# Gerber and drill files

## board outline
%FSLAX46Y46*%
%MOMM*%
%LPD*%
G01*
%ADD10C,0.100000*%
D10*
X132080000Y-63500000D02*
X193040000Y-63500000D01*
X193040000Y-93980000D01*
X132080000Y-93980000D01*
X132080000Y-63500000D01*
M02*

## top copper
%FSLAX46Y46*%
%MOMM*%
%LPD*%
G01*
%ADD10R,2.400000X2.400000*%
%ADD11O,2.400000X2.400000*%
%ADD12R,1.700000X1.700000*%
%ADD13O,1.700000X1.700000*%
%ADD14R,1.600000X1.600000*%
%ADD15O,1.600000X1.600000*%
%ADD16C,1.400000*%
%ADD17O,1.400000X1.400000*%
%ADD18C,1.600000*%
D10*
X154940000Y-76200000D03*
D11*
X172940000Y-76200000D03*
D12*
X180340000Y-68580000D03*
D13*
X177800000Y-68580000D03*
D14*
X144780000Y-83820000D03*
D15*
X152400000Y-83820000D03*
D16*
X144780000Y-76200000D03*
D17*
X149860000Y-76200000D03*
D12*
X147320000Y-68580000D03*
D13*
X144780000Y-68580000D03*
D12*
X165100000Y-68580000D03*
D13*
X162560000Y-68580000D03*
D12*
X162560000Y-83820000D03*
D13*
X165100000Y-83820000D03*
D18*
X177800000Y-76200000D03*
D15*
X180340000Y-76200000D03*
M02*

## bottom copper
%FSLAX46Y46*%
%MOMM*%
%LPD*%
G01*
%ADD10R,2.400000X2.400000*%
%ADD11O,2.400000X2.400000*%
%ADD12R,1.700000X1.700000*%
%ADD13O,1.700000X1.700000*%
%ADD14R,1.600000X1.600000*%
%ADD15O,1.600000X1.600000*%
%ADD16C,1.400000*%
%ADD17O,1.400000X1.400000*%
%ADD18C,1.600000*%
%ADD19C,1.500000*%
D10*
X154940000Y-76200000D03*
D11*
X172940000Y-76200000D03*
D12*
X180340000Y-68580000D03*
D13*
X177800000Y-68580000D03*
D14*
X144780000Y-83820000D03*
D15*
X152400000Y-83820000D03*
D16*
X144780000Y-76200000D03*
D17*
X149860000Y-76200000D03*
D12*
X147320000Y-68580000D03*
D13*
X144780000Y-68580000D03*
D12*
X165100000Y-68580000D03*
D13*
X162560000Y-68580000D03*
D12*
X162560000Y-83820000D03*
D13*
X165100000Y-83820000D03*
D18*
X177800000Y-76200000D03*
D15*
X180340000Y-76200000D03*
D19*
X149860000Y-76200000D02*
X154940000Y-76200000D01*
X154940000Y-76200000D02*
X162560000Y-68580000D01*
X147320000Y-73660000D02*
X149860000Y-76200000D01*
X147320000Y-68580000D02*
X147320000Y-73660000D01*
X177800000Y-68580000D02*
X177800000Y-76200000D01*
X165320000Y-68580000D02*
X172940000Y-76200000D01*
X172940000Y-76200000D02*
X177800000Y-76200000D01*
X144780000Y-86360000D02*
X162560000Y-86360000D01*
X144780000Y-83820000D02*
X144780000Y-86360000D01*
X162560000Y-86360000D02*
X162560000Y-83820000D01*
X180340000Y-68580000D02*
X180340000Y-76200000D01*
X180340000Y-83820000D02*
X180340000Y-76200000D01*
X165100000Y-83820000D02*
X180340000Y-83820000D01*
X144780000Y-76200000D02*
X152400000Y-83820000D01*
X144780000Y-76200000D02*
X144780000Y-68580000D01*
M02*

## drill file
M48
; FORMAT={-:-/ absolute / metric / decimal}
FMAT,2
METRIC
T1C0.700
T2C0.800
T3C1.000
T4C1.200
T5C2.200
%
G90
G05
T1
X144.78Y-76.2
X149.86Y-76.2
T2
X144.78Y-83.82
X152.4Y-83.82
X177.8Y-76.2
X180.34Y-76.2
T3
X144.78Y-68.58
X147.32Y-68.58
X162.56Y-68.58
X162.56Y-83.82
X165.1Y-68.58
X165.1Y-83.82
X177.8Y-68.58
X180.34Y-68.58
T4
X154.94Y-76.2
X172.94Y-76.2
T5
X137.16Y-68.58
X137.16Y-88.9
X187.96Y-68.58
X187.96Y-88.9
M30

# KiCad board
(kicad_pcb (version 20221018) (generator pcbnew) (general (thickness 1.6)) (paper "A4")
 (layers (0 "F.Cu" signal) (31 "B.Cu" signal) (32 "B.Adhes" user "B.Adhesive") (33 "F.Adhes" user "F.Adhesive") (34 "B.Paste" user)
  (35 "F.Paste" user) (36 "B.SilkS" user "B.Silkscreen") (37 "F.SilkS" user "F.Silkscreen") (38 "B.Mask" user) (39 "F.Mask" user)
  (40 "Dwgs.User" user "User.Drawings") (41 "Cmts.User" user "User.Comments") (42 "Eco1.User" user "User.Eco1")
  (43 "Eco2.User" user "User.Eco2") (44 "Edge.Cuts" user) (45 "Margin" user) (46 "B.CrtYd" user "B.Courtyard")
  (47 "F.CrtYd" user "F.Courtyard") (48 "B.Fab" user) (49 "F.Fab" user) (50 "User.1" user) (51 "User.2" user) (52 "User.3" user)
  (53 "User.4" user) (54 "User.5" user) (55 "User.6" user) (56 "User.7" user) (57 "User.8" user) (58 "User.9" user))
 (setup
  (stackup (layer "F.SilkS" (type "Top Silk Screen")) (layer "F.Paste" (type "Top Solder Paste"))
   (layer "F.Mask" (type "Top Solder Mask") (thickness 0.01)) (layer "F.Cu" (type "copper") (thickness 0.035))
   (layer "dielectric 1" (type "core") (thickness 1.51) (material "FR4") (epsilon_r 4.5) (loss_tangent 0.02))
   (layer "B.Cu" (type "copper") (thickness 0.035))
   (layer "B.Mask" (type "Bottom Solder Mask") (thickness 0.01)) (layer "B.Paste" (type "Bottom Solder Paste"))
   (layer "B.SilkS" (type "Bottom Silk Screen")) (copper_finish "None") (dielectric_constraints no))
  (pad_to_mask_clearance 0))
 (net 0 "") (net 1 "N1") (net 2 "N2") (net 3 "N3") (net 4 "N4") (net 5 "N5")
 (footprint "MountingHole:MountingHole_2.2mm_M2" (layer "F.Cu") (at 187.96 68.58)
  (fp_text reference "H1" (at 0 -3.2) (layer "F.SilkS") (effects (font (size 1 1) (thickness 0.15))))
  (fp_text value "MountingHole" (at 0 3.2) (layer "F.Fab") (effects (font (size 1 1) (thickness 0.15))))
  (pad "" np_thru_hole circle (at 0 0) (size 2.2 2.2) (drill 2.2) (layers "*.Cu" "*.Mask")))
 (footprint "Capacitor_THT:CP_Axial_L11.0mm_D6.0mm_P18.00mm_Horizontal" (layer "F.Cu") (at 154.94 76.2)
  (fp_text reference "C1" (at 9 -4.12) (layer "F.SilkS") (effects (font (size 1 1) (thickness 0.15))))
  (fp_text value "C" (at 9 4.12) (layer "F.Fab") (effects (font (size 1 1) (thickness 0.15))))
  (pad "1" thru_hole rect (at 0 0) (size 2.4 2.4) (drill 1.2) (layers "*.Cu" "*.Mask") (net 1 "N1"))
  (pad "2" thru_hole oval (at 18 0) (size 2.4 2.4) (drill 1.2) (layers "*.Cu" "*.Mask") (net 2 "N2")))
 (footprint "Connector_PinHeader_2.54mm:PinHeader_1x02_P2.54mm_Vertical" (layer "F.Cu") (at 180.34 68.58 -90)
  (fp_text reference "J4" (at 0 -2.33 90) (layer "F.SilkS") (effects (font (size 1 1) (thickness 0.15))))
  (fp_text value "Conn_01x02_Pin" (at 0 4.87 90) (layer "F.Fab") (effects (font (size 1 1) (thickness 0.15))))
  (pad "1" thru_hole rect (at 0 0 270) (size 1.7 1.7) (drill 1) (layers "*.Cu" "*.Mask") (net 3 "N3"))
  (pad "2" thru_hole oval (at 0 2.54 270) (size 1.7 1.7) (drill 1) (layers "*.Cu" "*.Mask") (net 2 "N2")))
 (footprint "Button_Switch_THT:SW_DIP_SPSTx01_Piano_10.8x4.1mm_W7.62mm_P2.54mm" (layer "F.Cu") (at 144.78 83.82)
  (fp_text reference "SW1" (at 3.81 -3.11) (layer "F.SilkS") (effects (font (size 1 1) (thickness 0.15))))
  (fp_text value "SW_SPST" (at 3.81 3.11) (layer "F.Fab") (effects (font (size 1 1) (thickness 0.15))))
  (pad "1" thru_hole rect (at 0 0) (size 1.6 1.6) (drill 0.8) (layers "*.Cu" "*.Mask") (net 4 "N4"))
  (pad "2" thru_hole oval (at 7.62 0) (size 1.6 1.6) (drill 0.8) (layers "*.Cu" "*.Mask") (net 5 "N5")))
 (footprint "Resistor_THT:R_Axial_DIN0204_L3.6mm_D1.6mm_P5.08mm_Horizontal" (layer "F.Cu") (at 144.78 76.2)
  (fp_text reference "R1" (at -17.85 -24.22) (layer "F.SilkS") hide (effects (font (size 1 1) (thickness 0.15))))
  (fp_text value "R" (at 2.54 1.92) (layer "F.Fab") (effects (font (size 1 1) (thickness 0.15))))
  (pad "1" thru_hole circle (at 0 0) (size 1.4 1.4) (drill 0.7) (layers "*.Cu" "*.Mask") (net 5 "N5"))
  (pad "2" thru_hole oval (at 5.08 0) (size 1.4 1.4) (drill 0.7) (layers "*.Cu" "*.Mask") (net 1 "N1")))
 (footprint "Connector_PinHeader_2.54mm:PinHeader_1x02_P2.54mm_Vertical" (layer "F.Cu") (at 147.32 68.58 -90)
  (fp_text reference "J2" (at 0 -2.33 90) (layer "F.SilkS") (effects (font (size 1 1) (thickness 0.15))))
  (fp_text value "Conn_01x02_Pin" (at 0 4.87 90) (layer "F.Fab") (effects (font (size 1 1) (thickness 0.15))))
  (pad "1" thru_hole rect (at 0 0 270) (size 1.7 1.7) (drill 1) (layers "*.Cu" "*.Mask") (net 1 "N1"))
  (pad "2" thru_hole oval (at 0 2.54 270) (size 1.7 1.7) (drill 1) (layers "*.Cu" "*.Mask") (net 5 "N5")))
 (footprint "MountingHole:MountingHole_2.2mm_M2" (layer "F.Cu") (at 187.96 88.9)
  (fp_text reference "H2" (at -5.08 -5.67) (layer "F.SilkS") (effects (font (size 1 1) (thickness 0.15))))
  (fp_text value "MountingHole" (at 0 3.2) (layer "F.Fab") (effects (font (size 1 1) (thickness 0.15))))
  (pad "" np_thru_hole circle (at 0 0) (size 2.2 2.2) (drill 2.2) (layers "*.Cu" "*.Mask")))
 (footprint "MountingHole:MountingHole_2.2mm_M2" (layer "F.Cu") (at 137.16 68.58)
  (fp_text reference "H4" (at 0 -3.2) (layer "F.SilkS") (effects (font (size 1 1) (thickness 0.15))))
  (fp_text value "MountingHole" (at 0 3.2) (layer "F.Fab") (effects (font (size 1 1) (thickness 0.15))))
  (pad "" np_thru_hole circle (at 0 0) (size 2.2 2.2) (drill 2.2) (layers "*.Cu" "*.Mask")))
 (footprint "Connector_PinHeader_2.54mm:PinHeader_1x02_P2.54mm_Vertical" (layer "F.Cu") (at 165.1 68.58 -90)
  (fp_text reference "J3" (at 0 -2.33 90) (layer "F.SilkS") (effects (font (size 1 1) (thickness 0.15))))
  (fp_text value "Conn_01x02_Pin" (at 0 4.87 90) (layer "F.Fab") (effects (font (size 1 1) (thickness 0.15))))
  (pad "1" thru_hole rect (at 0 0 270) (size 1.7 1.7) (drill 1) (layers "*.Cu" "*.Mask") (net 2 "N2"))
  (pad "2" thru_hole oval (at 0 2.54 270) (size 1.7 1.7) (drill 1) (layers "*.Cu" "*.Mask") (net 1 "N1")))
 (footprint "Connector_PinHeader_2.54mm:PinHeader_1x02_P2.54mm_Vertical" (layer "F.Cu") (at 162.56 83.82 90)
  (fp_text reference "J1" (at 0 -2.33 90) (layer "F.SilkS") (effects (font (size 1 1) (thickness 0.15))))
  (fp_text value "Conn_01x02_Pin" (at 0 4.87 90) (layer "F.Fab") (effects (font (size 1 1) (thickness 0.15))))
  (pad "1" thru_hole rect (at 0 0 90) (size 1.7 1.7) (drill 1) (layers "*.Cu" "*.Mask") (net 4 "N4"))
  (pad "2" thru_hole oval (at 0 2.54 90) (size 1.7 1.7) (drill 1) (layers "*.Cu" "*.Mask") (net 3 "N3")))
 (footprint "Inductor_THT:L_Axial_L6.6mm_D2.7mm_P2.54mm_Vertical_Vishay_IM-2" (layer "F.Cu") (at 177.8 76.2)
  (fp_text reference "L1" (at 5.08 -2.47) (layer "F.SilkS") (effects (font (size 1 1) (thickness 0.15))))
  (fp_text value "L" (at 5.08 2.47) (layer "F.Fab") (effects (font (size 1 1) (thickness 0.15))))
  (pad "1" thru_hole circle (at 0 0) (size 1.6 1.6) (drill 0.8) (layers "*.Cu" "*.Mask") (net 2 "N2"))
  (pad "2" thru_hole oval (at 2.54 0) (size 1.6 1.6) (drill 0.8) (layers "*.Cu" "*.Mask") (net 3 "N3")))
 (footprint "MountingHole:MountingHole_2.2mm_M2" (layer "F.Cu") (at 137.16 88.9)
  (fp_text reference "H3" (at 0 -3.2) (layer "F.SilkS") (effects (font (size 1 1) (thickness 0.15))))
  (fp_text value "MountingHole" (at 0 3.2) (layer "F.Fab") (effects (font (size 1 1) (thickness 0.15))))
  (pad "" np_thru_hole circle (at 0 0) (size 2.2 2.2) (drill 2.2) (layers "*.Cu" "*.Mask")))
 (gr_rect (start 132.08 63.5) (end 193.04 93.98) (stroke (width 0.1) (type default)) (fill none) (layer "Edge.Cuts"))
 (segment (start 149.86 76.2) (end 154.94 76.2) (width 1.5) (layer "B.Cu") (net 1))
 (segment (start 154.94 76.2) (end 162.56 68.58) (width 1.5) (layer "B.Cu") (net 1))
 (segment (start 147.32 73.66) (end 149.86 76.2) (width 1.5) (layer "B.Cu") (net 1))
 (segment (start 147.32 68.58) (end 147.32 73.66) (width 1.5) (layer "B.Cu") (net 1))
 (segment (start 177.8 68.58) (end 177.8 76.2) (width 1.5) (layer "B.Cu") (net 2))
 (segment (start 165.32 68.58) (end 172.94 76.2) (width 1.5) (layer "B.Cu") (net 2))
 (segment (start 172.94 76.2) (end 177.8 76.2) (width 1.5) (layer "B.Cu") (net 2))
 (segment (start 144.78 86.36) (end 162.56 86.36) (width 1.5) (layer "B.Cu") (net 4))
 (segment (start 144.78 83.82) (end 144.78 86.36) (width 1.5) (layer "B.Cu") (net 4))
 (segment (start 162.56 86.36) (end 162.56 83.82) (width 1.5) (layer "B.Cu") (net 4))
 (segment (start 180.34 68.58) (end 180.34 76.2) (width 1.5) (layer "B.Cu") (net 3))
 (segment (start 180.34 83.82) (end 180.34 76.2) (width 1.5) (layer "B.Cu") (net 3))
 (segment (start 165.1 83.82) (end 180.34 83.82) (width 1.5) (layer "B.Cu") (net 3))
 (segment (start 144.78 76.2) (end 152.4 83.82) (width 1.5) (layer "B.Cu") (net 5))
 (segment (start 144.78 76.2) (end 144.78 68.58) (width 1.5) (layer "B.Cu") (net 5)))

